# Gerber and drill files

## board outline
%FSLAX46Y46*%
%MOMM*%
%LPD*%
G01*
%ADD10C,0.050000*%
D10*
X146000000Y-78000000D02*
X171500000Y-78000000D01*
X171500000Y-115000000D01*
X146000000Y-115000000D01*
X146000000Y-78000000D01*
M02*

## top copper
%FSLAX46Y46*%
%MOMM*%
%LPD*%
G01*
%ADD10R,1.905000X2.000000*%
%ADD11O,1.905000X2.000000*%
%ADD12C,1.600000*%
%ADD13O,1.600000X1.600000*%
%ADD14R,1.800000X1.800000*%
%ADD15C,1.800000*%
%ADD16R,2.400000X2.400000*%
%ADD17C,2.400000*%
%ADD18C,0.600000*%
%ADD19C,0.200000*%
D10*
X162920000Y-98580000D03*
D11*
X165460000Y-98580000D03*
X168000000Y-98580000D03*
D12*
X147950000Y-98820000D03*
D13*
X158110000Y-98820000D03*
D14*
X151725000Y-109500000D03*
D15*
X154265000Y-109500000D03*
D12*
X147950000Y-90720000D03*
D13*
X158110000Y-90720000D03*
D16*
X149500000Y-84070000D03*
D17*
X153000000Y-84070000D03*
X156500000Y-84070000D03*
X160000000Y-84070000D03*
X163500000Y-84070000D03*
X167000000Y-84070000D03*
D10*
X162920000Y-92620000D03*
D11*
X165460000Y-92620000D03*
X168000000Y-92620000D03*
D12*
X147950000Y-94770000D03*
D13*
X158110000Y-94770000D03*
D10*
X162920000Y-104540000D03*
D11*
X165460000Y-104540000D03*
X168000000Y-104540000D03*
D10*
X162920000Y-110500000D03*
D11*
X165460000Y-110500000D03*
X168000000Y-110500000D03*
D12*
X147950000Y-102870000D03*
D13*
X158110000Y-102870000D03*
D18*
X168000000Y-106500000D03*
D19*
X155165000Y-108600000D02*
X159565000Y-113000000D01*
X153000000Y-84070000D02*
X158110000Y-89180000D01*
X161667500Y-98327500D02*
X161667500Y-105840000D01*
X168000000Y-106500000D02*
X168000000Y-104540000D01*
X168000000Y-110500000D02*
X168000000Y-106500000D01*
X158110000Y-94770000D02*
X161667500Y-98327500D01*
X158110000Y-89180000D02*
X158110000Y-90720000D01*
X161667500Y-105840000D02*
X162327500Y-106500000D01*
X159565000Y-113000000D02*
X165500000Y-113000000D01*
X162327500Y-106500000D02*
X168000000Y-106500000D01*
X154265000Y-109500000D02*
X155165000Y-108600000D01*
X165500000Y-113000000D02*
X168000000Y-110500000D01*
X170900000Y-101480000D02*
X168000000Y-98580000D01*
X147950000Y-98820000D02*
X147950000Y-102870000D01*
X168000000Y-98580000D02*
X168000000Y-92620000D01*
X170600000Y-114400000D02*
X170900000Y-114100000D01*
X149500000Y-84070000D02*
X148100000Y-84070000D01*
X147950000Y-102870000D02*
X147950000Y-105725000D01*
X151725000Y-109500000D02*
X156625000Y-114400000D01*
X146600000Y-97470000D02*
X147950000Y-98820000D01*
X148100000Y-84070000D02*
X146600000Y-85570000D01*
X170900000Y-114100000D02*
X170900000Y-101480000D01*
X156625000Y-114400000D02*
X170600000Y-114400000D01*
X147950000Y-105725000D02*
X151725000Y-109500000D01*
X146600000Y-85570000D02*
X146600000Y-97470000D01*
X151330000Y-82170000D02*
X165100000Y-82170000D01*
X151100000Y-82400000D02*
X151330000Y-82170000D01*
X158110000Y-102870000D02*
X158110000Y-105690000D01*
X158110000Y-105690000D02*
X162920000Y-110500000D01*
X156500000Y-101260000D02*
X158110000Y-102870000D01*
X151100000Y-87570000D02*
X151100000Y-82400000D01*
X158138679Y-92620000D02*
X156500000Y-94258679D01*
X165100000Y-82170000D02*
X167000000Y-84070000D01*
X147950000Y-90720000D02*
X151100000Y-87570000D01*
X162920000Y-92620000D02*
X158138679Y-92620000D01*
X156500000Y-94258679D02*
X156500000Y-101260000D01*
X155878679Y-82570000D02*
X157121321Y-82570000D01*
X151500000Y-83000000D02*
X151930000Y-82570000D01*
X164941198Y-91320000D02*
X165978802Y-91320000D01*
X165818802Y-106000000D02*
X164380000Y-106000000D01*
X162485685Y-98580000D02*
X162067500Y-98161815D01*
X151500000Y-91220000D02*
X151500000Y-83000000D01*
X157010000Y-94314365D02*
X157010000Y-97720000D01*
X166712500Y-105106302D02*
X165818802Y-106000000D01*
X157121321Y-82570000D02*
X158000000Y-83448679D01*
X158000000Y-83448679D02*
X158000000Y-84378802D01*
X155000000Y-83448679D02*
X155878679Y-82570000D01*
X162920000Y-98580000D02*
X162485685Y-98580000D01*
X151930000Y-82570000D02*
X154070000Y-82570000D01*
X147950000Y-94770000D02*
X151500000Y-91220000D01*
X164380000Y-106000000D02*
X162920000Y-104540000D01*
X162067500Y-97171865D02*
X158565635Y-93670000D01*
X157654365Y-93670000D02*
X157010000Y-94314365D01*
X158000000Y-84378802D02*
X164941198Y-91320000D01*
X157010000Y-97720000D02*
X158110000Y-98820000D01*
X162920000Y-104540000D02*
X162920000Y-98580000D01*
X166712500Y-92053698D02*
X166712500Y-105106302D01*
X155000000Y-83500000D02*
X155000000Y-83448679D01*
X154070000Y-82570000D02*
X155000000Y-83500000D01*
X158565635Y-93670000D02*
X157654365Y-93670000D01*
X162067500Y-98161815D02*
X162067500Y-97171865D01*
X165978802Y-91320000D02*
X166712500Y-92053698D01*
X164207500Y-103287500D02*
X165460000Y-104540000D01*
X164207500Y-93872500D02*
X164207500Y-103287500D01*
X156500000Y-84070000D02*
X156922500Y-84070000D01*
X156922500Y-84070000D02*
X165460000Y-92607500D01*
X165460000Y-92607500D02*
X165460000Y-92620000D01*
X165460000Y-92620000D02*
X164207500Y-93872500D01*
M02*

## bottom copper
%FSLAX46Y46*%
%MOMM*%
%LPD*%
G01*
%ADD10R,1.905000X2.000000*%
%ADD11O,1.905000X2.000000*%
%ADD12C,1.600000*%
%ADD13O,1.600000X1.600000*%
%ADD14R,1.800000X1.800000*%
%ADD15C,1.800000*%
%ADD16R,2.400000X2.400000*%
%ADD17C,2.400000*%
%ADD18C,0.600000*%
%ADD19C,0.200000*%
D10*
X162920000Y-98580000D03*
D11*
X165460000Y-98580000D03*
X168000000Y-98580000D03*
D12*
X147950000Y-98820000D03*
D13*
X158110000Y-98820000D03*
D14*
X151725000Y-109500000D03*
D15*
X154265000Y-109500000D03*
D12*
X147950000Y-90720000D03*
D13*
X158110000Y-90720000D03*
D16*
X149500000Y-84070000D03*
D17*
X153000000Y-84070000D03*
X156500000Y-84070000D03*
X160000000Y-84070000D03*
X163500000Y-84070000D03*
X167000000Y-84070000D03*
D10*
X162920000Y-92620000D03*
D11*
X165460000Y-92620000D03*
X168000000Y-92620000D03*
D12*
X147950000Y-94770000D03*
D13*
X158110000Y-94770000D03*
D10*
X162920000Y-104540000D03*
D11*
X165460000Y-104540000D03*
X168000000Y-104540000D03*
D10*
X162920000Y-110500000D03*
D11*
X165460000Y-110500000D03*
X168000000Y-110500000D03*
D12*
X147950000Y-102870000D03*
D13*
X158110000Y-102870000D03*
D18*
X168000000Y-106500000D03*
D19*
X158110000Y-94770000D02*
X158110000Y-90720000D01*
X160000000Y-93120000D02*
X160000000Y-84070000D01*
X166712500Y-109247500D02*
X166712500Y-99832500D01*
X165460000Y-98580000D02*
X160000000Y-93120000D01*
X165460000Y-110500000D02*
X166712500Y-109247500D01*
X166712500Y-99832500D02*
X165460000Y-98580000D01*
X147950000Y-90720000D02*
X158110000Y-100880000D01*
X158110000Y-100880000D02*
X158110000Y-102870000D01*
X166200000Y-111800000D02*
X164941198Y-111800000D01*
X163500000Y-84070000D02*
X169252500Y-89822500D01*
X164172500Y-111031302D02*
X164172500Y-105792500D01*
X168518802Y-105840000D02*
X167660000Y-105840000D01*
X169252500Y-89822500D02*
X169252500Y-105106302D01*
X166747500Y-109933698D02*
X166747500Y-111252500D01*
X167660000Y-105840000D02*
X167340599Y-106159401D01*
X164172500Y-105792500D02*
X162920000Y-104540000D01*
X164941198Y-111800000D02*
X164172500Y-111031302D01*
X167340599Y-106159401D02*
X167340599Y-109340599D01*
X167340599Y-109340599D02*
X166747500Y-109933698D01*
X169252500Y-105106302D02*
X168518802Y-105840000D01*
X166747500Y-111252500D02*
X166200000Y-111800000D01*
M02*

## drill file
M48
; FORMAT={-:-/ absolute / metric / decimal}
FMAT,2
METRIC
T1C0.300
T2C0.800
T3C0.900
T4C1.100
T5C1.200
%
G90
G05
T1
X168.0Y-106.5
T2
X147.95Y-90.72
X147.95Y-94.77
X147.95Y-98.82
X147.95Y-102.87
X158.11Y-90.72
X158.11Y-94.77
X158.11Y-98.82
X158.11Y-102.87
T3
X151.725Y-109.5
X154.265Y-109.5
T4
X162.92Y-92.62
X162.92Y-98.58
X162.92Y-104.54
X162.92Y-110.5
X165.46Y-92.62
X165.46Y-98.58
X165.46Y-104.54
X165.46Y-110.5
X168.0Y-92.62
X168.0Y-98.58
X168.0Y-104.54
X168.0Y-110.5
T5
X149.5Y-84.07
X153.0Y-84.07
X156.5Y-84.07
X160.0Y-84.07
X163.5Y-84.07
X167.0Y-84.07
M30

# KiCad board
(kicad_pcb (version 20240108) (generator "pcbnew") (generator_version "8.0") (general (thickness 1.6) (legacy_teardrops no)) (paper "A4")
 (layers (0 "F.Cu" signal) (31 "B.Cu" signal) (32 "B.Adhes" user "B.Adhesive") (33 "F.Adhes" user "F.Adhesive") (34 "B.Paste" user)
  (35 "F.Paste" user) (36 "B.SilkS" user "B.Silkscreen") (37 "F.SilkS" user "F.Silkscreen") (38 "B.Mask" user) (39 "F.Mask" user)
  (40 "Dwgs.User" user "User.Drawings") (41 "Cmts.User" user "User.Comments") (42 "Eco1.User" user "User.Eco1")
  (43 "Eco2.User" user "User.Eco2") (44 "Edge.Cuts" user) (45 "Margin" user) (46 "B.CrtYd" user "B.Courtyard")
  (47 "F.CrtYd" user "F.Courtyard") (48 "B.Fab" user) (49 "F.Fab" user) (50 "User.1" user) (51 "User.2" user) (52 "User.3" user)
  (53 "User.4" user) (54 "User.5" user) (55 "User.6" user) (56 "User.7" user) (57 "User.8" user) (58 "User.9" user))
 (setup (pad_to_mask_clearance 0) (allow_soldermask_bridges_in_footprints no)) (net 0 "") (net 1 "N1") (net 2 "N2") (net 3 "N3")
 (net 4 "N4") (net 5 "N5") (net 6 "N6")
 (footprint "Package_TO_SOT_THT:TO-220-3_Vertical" (layer "F.Cu") (at 162.92 98.58)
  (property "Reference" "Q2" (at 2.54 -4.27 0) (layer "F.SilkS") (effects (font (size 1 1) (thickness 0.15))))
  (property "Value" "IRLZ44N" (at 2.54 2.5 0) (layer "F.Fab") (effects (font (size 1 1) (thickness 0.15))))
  (pad "1" thru_hole rect (at 0 0) (size 1.905 2) (drill 1.1) (layers "*.Cu" "*.Mask") (remove_unused_layers no) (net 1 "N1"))
  (pad "2" thru_hole oval (at 2.54 0) (size 1.905 2) (drill 1.1) (layers "*.Cu" "*.Mask") (remove_unused_layers no) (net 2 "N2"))
  (pad "3" thru_hole oval (at 5.08 0) (size 1.905 2) (drill 1.1) (layers "*.Cu" "*.Mask") (remove_unused_layers no) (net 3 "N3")))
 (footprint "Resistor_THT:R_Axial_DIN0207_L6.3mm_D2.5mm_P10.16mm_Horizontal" (layer "F.Cu") (at 147.95 98.82)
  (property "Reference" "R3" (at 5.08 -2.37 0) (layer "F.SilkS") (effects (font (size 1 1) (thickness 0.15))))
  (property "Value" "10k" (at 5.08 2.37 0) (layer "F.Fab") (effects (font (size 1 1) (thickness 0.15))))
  (pad "1" thru_hole circle (at 0 0) (size 1.6 1.6) (drill 0.8) (layers "*.Cu" "*.Mask") (remove_unused_layers no) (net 3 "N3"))
  (pad "2" thru_hole oval (at 10.16 0) (size 1.6 1.6) (drill 0.8) (layers "*.Cu" "*.Mask") (remove_unused_layers no) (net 1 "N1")))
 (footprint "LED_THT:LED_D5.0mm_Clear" (layer "F.Cu") (at 151.725 109.5)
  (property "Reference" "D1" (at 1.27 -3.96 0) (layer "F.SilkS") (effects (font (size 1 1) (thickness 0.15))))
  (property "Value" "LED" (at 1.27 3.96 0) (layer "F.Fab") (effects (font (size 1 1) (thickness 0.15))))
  (pad "1" thru_hole rect (at 0 0) (size 1.8 1.8) (drill 0.9) (layers "*.Cu" "*.Mask") (remove_unused_layers no) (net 3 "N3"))
  (pad "2" thru_hole circle (at 2.54 0) (size 1.8 1.8) (drill 0.9) (layers "*.Cu" "*.Mask") (remove_unused_layers no) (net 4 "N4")))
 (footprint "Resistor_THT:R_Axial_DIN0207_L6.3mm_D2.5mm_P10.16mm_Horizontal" (layer "F.Cu") (at 147.95 90.72)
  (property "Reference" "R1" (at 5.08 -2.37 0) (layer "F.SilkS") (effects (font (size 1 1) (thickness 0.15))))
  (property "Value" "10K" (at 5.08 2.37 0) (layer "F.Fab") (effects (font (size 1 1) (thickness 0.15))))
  (pad "1" thru_hole circle (at 0 0) (size 1.6 1.6) (drill 0.8) (layers "*.Cu" "*.Mask") (remove_unused_layers no) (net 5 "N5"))
  (pad "2" thru_hole oval (at 10.16 0) (size 1.6 1.6) (drill 0.8) (layers "*.Cu" "*.Mask") (remove_unused_layers no) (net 4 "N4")))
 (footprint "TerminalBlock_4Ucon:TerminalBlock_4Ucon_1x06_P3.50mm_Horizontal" (layer "F.Cu") (at 149.5 84.07)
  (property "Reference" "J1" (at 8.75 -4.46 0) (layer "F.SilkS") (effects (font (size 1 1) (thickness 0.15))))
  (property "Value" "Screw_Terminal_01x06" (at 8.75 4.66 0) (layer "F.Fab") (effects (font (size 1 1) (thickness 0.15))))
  (pad "1" thru_hole rect (at 0 0) (size 2.4 2.4) (drill 1.2) (layers "*.Cu" "*.Mask") (remove_unused_layers no) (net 3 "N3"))
  (pad "2" thru_hole circle (at 3.5 0) (size 2.4 2.4) (drill 1.2) (layers "*.Cu" "*.Mask") (remove_unused_layers no) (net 4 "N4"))
  (pad "3" thru_hole circle (at 7 0) (size 2.4 2.4) (drill 1.2) (layers "*.Cu" "*.Mask") (remove_unused_layers no) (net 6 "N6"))
  (pad "4" thru_hole circle (at 10.5 0) (size 2.4 2.4) (drill 1.2) (layers "*.Cu" "*.Mask") (remove_unused_layers no) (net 2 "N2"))
  (pad "5" thru_hole circle (at 14 0) (size 2.4 2.4) (drill 1.2) (layers "*.Cu" "*.Mask") (remove_unused_layers no) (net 1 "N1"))
  (pad "6" thru_hole circle (at 17.5 0) (size 2.4 2.4) (drill 1.2) (layers "*.Cu" "*.Mask") (remove_unused_layers no) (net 5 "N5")))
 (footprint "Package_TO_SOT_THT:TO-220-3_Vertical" (layer "F.Cu") (at 162.92 92.62)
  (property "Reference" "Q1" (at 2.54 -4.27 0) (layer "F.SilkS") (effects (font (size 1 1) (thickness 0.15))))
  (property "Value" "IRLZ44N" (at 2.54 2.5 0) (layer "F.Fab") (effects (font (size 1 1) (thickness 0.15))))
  (pad "1" thru_hole rect (at 0 0) (size 1.905 2) (drill 1.1) (layers "*.Cu" "*.Mask") (remove_unused_layers no) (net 5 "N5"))
  (pad "2" thru_hole oval (at 2.54 0) (size 1.905 2) (drill 1.1) (layers "*.Cu" "*.Mask") (remove_unused_layers no) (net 6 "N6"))
  (pad "3" thru_hole oval (at 5.08 0) (size 1.905 2) (drill 1.1) (layers "*.Cu" "*.Mask") (remove_unused_layers no) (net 3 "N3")))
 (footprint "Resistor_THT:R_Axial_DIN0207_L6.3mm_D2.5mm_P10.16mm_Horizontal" (layer "F.Cu") (at 147.95 94.77)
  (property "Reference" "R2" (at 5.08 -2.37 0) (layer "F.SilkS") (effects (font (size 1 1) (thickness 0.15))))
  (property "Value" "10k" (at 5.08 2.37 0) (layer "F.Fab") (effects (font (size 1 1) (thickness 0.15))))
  (pad "1" thru_hole circle (at 0 0) (size 1.6 1.6) (drill 0.8) (layers "*.Cu" "*.Mask") (remove_unused_layers no) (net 1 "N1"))
  (pad "2" thru_hole oval (at 10.16 0) (size 1.6 1.6) (drill 0.8) (layers "*.Cu" "*.Mask") (remove_unused_layers no) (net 4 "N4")))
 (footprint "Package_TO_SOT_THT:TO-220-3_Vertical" (layer "F.Cu") (at 162.92 104.54)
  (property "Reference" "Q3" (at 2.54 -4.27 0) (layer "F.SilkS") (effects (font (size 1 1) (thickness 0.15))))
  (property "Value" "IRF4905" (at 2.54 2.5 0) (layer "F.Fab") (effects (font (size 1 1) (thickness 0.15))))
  (pad "1" thru_hole rect (at 0 0) (size 1.905 2) (drill 1.1) (layers "*.Cu" "*.Mask") (remove_unused_layers no) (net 1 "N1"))
  (pad "2" thru_hole oval (at 2.54 0) (size 1.905 2) (drill 1.1) (layers "*.Cu" "*.Mask") (remove_unused_layers no) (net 6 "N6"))
  (pad "3" thru_hole oval (at 5.08 0) (size 1.905 2) (drill 1.1) (layers "*.Cu" "*.Mask") (remove_unused_layers no) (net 4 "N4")))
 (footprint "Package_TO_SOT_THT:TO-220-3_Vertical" (layer "F.Cu") (at 162.92 110.5)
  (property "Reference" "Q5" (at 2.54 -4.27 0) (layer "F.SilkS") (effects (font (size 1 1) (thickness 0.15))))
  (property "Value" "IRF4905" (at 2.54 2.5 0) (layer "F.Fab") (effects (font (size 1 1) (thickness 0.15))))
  (pad "1" thru_hole rect (at 0 0) (size 1.905 2) (drill 1.1) (layers "*.Cu" "*.Mask") (remove_unused_layers no) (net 5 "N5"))
  (pad "2" thru_hole oval (at 2.54 0) (size 1.905 2) (drill 1.1) (layers "*.Cu" "*.Mask") (remove_unused_layers no) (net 2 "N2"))
  (pad "3" thru_hole oval (at 5.08 0) (size 1.905 2) (drill 1.1) (layers "*.Cu" "*.Mask") (remove_unused_layers no) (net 4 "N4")))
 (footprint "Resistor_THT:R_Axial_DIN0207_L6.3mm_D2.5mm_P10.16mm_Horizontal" (layer "F.Cu") (at 147.95 102.87)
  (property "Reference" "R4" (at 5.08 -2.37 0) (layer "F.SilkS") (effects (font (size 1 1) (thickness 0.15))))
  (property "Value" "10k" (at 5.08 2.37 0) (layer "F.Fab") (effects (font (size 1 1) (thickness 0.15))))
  (pad "1" thru_hole circle (at 0 0) (size 1.6 1.6) (drill 0.8) (layers "*.Cu" "*.Mask") (remove_unused_layers no) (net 3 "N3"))
  (pad "2" thru_hole oval (at 10.16 0) (size 1.6 1.6) (drill 0.8) (layers "*.Cu" "*.Mask") (remove_unused_layers no) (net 5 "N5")))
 (gr_rect (start 146 78) (end 171.5 115) (stroke (width 0.05) (type default)) (fill none) (layer "Edge.Cuts"))
 (segment (start 155.165 108.6) (end 159.565 113) (width 0.2) (layer "F.Cu") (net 4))
 (segment (start 153 84.07) (end 158.11 89.18) (width 0.2) (layer "F.Cu") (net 4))
 (segment (start 161.6675 98.3275) (end 161.6675 105.84) (width 0.2) (layer "F.Cu") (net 4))
 (segment (start 168 106.5) (end 168 104.54) (width 0.2) (layer "F.Cu") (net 4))
 (segment (start 168 110.5) (end 168 106.5) (width 0.2) (layer "F.Cu") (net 4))
 (segment (start 158.11 94.77) (end 161.6675 98.3275) (width 0.2) (layer "F.Cu") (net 4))
 (segment (start 158.11 89.18) (end 158.11 90.72) (width 0.2) (layer "F.Cu") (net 4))
 (segment (start 161.6675 105.84) (end 162.3275 106.5) (width 0.2) (layer "F.Cu") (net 4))
 (segment (start 159.565 113) (end 165.5 113) (width 0.2) (layer "F.Cu") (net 4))
 (segment (start 162.3275 106.5) (end 168 106.5) (width 0.2) (layer "F.Cu") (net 4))
 (segment (start 154.265 109.5) (end 155.165 108.6) (width 0.2) (layer "F.Cu") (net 4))
 (segment (start 165.5 113) (end 168 110.5) (width 0.2) (layer "F.Cu") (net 4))
 (via (at 168 106.5) (size 0.6) (drill 0.3) (layers "F.Cu" "B.Cu") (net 4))
 (segment (start 158.11 94.77) (end 158.11 90.72) (width 0.2) (layer "B.Cu") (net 4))
 (segment (start 170.9 101.48) (end 168 98.58) (width 0.2) (layer "F.Cu") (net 3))
 (segment (start 147.95 98.82) (end 147.95 102.87) (width 0.2) (layer "F.Cu") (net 3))
 (segment (start 168 98.58) (end 168 92.62) (width 0.2) (layer "F.Cu") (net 3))
 (segment (start 170.6 114.4) (end 170.9 114.1) (width 0.2) (layer "F.Cu") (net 3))
 (segment (start 149.5 84.07) (end 148.1 84.07) (width 0.2) (layer "F.Cu") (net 3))
 (segment (start 147.95 102.87) (end 147.95 105.725) (width 0.2) (layer "F.Cu") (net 3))
 (segment (start 151.725 109.5) (end 156.625 114.4) (width 0.2) (layer "F.Cu") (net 3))
 (segment (start 146.6 97.47) (end 147.95 98.82) (width 0.2) (layer "F.Cu") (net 3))
 (segment (start 148.1 84.07) (end 146.6 85.57) (width 0.2) (layer "F.Cu") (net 3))
 (segment (start 170.9 114.1) (end 170.9 101.48) (width 0.2) (layer "F.Cu") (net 3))
 (segment (start 156.625 114.4) (end 170.6 114.4) (width 0.2) (layer "F.Cu") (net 3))
 (segment (start 147.95 105.725) (end 151.725 109.5) (width 0.2) (layer "F.Cu") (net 3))
 (segment (start 146.6 85.57) (end 146.6 97.47) (width 0.2) (layer "F.Cu") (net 3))
 (segment (start 160 93.12) (end 160 84.07) (width 0.2) (layer "B.Cu") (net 2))
 (segment (start 166.7125 109.2475) (end 166.7125 99.8325) (width 0.2) (layer "B.Cu") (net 2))
 (segment (start 165.46 98.58) (end 160 93.12) (width 0.2) (layer "B.Cu") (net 2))
 (segment (start 165.46 110.5) (end 166.7125 109.2475) (width 0.2) (layer "B.Cu") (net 2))
 (segment (start 166.7125 99.8325) (end 165.46 98.58) (width 0.2) (layer "B.Cu") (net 2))
 (segment (start 151.33 82.17) (end 165.1 82.17) (width 0.2) (layer "F.Cu") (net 5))
 (segment (start 151.1 82.4) (end 151.33 82.17) (width 0.2) (layer "F.Cu") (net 5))
 (segment (start 158.11 102.87) (end 158.11 105.69) (width 0.2) (layer "F.Cu") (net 5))
 (segment (start 158.11 105.69) (end 162.92 110.5) (width 0.2) (layer "F.Cu") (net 5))
 (segment (start 156.5 101.26) (end 158.11 102.87) (width 0.2) (layer "F.Cu") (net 5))
 (segment (start 151.1 87.57) (end 151.1 82.4) (width 0.2) (layer "F.Cu") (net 5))
 (segment (start 158.138679 92.62) (end 156.5 94.258679) (width 0.2) (layer "F.Cu") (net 5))
 (segment (start 165.1 82.17) (end 167 84.07) (width 0.2) (layer "F.Cu") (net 5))
 (segment (start 147.95 90.72) (end 151.1 87.57) (width 0.2) (layer "F.Cu") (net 5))
 (segment (start 162.92 92.62) (end 158.138679 92.62) (width 0.2) (layer "F.Cu") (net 5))
 (segment (start 156.5 94.258679) (end 156.5 101.26) (width 0.2) (layer "F.Cu") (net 5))
 (segment (start 147.95 90.72) (end 158.11 100.88) (width 0.2) (layer "B.Cu") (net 5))
 (segment (start 158.11 100.88) (end 158.11 102.87) (width 0.2) (layer "B.Cu") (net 5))
 (segment (start 155.878679 82.57) (end 157.121321 82.57) (width 0.2) (layer "F.Cu") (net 1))
 (segment (start 151.5 83) (end 151.93 82.57) (width 0.2) (layer "F.Cu") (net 1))
 (segment (start 164.941198 91.32) (end 165.978802 91.32) (width 0.2) (layer "F.Cu") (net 1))
 (segment (start 165.818802 106) (end 164.38 106) (width 0.2) (layer "F.Cu") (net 1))
 (segment (start 162.485685 98.58) (end 162.0675 98.161815) (width 0.2) (layer "F.Cu") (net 1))
 (segment (start 151.5 91.22) (end 151.5 83) (width 0.2) (layer "F.Cu") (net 1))
 (segment (start 157.01 94.314365) (end 157.01 97.72) (width 0.2) (layer "F.Cu") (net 1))
 (segment (start 166.7125 105.106302) (end 165.818802 106) (width 0.2) (layer "F.Cu") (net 1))
 (segment (start 157.121321 82.57) (end 158 83.448679) (width 0.2) (layer "F.Cu") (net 1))
 (segment (start 158 83.448679) (end 158 84.378802) (width 0.2) (layer "F.Cu") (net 1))
 (segment (start 155 83.448679) (end 155.878679 82.57) (width 0.2) (layer "F.Cu") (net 1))
 (segment (start 162.92 98.58) (end 162.485685 98.58) (width 0.2) (layer "F.Cu") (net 1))
 (segment (start 151.93 82.57) (end 154.07 82.57) (width 0.2) (layer "F.Cu") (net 1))
 (segment (start 147.95 94.77) (end 151.5 91.22) (width 0.2) (layer "F.Cu") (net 1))
 (segment (start 164.38 106) (end 162.92 104.54) (width 0.2) (layer "F.Cu") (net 1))
 (segment (start 162.0675 97.171865) (end 158.565635 93.67) (width 0.2) (layer "F.Cu") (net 1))
 (segment (start 157.654365 93.67) (end 157.01 94.314365) (width 0.2) (layer "F.Cu") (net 1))
 (segment (start 158 84.378802) (end 164.941198 91.32) (width 0.2) (layer "F.Cu") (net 1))
 (segment (start 157.01 97.72) (end 158.11 98.82) (width 0.2) (layer "F.Cu") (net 1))
 (segment (start 162.92 104.54) (end 162.92 98.58) (width 0.2) (layer "F.Cu") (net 1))
 (segment (start 166.7125 92.053698) (end 166.7125 105.106302) (width 0.2) (layer "F.Cu") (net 1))
 (segment (start 155 83.5) (end 155 83.448679) (width 0.2) (layer "F.Cu") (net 1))
 (segment (start 154.07 82.57) (end 155 83.5) (width 0.2) (layer "F.Cu") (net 1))
 (segment (start 158.565635 93.67) (end 157.654365 93.67) (width 0.2) (layer "F.Cu") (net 1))
 (segment (start 162.0675 98.161815) (end 162.0675 97.171865) (width 0.2) (layer "F.Cu") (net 1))
 (segment (start 165.978802 91.32) (end 166.7125 92.053698) (width 0.2) (layer "F.Cu") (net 1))
 (segment (start 166.2 111.8) (end 164.941198 111.8) (width 0.2) (layer "B.Cu") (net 1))
 (segment (start 163.5 84.07) (end 169.2525 89.8225) (width 0.2) (layer "B.Cu") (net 1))
 (segment (start 164.1725 111.031302) (end 164.1725 105.7925) (width 0.2) (layer "B.Cu") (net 1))
 (segment (start 168.518802 105.84) (end 167.66 105.84) (width 0.2) (layer "B.Cu") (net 1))
 (segment (start 169.2525 89.8225) (end 169.2525 105.106302) (width 0.2) (layer "B.Cu") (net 1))
 (segment (start 166.7475 109.933698) (end 166.7475 111.2525) (width 0.2) (layer "B.Cu") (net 1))
 (segment (start 167.66 105.84) (end 167.340599 106.159401) (width 0.2) (layer "B.Cu") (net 1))
 (segment (start 164.1725 105.7925) (end 162.92 104.54) (width 0.2) (layer "B.Cu") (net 1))
 (segment (start 164.941198 111.8) (end 164.1725 111.031302) (width 0.2) (layer "B.Cu") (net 1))
 (segment (start 167.340599 106.159401) (end 167.340599 109.340599) (width 0.2) (layer "B.Cu") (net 1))
 (segment (start 167.340599 109.340599) (end 166.7475 109.933698) (width 0.2) (layer "B.Cu") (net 1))
 (segment (start 169.2525 105.106302) (end 168.518802 105.84) (width 0.2) (layer "B.Cu") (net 1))
 (segment (start 166.7475 111.2525) (end 166.2 111.8) (width 0.2) (layer "B.Cu") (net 1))
 (segment (start 164.2075 103.2875) (end 165.46 104.54) (width 0.2) (layer "F.Cu") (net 6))
 (segment (start 164.2075 93.8725) (end 164.2075 103.2875) (width 0.2) (layer "F.Cu") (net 6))
 (segment (start 156.5 84.07) (end 156.9225 84.07) (width 0.2) (layer "F.Cu") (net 6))
 (segment (start 156.9225 84.07) (end 165.46 92.6075) (width 0.2) (layer "F.Cu") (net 6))
 (segment (start 165.46 92.6075) (end 165.46 92.62) (width 0.2) (layer "F.Cu") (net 6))
 (segment (start 165.46 92.62) (end 164.2075 93.8725) (width 0.2) (layer "F.Cu") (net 6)))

